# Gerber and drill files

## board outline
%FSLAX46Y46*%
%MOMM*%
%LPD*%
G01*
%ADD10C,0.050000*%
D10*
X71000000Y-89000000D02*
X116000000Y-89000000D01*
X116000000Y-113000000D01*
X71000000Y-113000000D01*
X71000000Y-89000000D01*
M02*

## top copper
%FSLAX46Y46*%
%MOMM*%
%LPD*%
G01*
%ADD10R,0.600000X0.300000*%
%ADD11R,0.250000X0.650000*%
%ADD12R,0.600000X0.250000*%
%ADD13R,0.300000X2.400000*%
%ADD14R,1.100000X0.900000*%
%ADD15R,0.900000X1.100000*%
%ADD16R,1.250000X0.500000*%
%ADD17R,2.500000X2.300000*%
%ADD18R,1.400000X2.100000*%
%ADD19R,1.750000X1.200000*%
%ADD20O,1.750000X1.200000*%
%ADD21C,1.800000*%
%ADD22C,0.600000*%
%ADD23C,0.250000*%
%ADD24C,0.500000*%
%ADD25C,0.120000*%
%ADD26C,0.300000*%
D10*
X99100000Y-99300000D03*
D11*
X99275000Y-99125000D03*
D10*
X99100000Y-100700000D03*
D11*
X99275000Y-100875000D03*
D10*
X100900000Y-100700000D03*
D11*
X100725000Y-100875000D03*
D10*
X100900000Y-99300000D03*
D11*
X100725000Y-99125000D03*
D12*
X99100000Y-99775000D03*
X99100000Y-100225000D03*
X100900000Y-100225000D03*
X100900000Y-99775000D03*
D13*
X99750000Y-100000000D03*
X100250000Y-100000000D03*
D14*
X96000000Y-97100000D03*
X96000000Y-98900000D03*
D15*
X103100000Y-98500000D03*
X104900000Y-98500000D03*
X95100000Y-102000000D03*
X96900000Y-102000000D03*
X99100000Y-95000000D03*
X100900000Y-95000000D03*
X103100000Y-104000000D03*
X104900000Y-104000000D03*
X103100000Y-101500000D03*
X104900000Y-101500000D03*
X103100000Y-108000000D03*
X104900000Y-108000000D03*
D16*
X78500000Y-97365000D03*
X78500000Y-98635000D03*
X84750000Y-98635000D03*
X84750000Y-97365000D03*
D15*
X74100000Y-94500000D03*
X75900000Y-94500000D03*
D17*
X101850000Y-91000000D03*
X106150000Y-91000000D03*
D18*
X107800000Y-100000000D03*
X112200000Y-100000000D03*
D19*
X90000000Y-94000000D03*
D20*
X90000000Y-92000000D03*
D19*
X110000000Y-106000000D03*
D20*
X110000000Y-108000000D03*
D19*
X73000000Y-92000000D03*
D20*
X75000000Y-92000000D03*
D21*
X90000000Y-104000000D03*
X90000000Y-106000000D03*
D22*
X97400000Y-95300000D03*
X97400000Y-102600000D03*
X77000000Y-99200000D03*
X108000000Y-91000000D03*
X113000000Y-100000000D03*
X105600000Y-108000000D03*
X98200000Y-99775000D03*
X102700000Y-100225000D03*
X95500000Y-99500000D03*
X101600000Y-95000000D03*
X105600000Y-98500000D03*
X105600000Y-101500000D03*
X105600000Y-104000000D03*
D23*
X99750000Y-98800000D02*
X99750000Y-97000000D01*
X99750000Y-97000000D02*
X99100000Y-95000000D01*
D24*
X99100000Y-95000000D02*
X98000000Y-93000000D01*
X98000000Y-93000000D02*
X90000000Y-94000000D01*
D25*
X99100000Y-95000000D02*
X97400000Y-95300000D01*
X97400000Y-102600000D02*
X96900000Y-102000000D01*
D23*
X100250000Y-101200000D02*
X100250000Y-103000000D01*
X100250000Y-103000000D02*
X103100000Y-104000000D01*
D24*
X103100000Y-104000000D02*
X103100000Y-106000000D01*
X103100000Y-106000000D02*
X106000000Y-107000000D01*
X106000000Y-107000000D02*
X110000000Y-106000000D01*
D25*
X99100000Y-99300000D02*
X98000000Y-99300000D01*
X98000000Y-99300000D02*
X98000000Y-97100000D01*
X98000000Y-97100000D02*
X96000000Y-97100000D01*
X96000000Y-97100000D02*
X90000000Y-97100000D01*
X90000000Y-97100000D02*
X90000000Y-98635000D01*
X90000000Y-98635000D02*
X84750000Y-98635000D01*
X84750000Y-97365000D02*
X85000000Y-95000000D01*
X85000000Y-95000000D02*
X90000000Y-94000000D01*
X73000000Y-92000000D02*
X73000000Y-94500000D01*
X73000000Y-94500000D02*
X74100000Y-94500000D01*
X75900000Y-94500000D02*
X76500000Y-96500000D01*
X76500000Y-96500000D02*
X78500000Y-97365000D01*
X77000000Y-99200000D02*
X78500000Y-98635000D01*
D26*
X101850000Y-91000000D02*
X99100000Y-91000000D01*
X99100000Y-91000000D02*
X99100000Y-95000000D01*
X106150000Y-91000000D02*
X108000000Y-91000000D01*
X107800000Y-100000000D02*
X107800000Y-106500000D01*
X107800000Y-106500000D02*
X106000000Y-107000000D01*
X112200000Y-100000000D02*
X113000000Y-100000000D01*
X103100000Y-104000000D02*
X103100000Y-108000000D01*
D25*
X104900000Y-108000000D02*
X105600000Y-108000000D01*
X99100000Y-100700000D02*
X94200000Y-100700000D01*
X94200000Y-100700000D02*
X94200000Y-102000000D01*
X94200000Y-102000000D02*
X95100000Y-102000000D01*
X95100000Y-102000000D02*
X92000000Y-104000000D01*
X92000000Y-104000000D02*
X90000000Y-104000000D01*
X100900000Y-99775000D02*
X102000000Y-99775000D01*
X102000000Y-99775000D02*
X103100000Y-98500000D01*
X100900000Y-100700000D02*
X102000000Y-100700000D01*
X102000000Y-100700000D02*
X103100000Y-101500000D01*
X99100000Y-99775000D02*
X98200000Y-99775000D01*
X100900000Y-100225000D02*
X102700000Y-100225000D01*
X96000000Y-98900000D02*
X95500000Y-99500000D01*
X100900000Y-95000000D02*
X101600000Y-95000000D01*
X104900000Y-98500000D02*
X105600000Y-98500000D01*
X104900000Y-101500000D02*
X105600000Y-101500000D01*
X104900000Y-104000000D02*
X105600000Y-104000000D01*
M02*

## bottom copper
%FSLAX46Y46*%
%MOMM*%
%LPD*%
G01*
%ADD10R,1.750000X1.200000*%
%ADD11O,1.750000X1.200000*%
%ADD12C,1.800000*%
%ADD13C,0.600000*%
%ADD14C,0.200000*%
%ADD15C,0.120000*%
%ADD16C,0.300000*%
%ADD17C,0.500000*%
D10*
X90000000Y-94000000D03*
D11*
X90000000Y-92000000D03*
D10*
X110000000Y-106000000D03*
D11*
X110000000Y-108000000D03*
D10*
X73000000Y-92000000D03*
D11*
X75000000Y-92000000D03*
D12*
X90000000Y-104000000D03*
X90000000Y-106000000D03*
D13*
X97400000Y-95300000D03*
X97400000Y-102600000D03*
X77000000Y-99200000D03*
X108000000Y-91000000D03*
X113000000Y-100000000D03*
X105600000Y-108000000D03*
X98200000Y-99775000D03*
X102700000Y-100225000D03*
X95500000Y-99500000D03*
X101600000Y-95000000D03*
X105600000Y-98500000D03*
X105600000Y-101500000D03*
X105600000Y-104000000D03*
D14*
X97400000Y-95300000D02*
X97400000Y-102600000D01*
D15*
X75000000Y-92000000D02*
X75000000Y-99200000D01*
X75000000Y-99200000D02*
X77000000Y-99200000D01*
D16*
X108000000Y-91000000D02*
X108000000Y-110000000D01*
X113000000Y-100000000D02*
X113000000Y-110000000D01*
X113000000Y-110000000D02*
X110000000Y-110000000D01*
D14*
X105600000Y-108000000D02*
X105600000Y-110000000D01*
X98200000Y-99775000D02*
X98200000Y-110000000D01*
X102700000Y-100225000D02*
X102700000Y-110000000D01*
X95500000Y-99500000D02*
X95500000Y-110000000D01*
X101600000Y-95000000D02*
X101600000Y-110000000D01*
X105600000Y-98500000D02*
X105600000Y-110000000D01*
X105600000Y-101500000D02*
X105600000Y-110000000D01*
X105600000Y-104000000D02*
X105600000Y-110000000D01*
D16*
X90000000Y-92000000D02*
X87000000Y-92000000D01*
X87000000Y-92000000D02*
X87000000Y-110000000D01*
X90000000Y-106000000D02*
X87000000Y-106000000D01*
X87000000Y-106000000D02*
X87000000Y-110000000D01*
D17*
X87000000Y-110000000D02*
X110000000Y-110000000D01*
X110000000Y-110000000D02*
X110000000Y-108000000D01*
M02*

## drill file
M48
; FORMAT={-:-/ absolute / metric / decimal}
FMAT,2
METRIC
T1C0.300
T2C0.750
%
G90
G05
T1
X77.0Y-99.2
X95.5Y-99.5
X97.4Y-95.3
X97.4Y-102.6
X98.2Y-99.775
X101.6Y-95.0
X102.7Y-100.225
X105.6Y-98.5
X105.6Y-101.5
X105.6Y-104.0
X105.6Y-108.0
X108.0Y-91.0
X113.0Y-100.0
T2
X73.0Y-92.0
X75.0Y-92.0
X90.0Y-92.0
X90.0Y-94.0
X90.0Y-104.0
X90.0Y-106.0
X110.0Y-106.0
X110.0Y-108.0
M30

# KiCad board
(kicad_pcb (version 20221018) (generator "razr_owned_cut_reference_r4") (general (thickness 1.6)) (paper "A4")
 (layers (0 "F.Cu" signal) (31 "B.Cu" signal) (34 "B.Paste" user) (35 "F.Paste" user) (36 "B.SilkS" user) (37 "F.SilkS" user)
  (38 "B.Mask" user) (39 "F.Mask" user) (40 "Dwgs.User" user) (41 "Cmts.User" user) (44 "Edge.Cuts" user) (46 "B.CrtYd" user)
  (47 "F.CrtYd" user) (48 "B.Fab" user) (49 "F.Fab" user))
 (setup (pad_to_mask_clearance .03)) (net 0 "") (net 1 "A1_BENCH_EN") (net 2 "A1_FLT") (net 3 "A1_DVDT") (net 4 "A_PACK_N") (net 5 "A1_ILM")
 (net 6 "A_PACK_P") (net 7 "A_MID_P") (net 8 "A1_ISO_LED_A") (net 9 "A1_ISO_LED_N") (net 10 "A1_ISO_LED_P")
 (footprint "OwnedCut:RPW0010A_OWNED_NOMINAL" (layer "F.Cu") (at 100 100)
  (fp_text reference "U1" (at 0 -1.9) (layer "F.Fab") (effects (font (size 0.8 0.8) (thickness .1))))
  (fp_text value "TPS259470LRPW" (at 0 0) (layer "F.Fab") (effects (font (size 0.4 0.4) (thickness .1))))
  (pad "1" smd rect (at -0.9 -0.7) (size 0.6 0.3) (layers "F.Cu" "F.Paste" "F.Mask") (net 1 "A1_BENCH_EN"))
  (pad "1" smd rect (at -0.725 -0.875) (size 0.25 0.65) (layers "F.Cu" "F.Paste" "F.Mask") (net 1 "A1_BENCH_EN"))
  (pad "4" smd rect (at -0.9 0.7) (size 0.6 0.3) (layers "F.Cu" "F.Paste" "F.Mask") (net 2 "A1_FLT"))
  (pad "4" smd rect (at -0.725 0.875) (size 0.25 0.65) (layers "F.Cu" "F.Paste" "F.Mask") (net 2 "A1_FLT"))
  (pad "7" smd rect (at 0.9 0.7) (size 0.6 0.3) (layers "F.Cu" "F.Paste" "F.Mask") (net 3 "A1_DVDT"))
  (pad "7" smd rect (at 0.725 0.875) (size 0.25 0.65) (layers "F.Cu" "F.Paste" "F.Mask") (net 3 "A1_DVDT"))
  (pad "10" smd rect (at 0.9 -0.7) (size 0.6 0.3) (layers "F.Cu" "F.Paste" "F.Mask"))
  (pad "10" smd rect (at 0.725 -0.875) (size 0.25 0.65) (layers "F.Cu" "F.Paste" "F.Mask"))
  (pad "2" smd rect (at -0.9 -0.225) (size 0.6 0.25) (layers "F.Cu" "F.Paste" "F.Mask") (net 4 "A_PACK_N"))
  (pad "3" smd rect (at -0.9 0.225) (size 0.6 0.25) (layers "F.Cu" "F.Paste" "F.Mask"))
  (pad "8" smd rect (at 0.9 0.225) (size 0.6 0.25) (layers "F.Cu" "F.Paste" "F.Mask") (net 4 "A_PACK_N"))
  (pad "9" smd rect (at 0.9 -0.225) (size 0.6 0.25) (layers "F.Cu" "F.Paste" "F.Mask") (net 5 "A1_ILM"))
  (pad "5" smd rect (at -0.25 0) (size 0.3 2.4) (layers "F.Cu" "F.Paste" "F.Mask") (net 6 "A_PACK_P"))
  (pad "6" smd rect (at 0.25 0) (size 0.3 2.4) (layers "F.Cu" "F.Paste" "F.Mask") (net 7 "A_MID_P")))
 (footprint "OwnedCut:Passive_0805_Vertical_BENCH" (layer "F.Cu") (at 96 98)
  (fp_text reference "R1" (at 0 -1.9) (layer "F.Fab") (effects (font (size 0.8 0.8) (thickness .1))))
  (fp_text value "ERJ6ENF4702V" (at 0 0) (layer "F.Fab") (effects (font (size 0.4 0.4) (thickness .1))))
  (pad "1" smd rect (at 0 -0.9) (size 1.1 0.9) (layers "F.Cu" "F.Paste" "F.Mask") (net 1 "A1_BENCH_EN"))
  (pad "2" smd rect (at 0 0.9) (size 1.1 0.9) (layers "F.Cu" "F.Paste" "F.Mask") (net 4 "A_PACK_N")))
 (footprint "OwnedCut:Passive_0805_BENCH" (layer "F.Cu") (at 104 98.5)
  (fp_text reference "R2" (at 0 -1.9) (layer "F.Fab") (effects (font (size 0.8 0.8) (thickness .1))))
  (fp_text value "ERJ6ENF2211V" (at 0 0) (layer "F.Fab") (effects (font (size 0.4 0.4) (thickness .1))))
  (pad "1" smd rect (at -0.9 0) (size 0.9 1.1) (layers "F.Cu" "F.Paste" "F.Mask") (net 5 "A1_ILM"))
  (pad "2" smd rect (at 0.9 0) (size 0.9 1.1) (layers "F.Cu" "F.Paste" "F.Mask") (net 4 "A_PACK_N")))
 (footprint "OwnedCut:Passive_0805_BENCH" (layer "F.Cu") (at 96 102)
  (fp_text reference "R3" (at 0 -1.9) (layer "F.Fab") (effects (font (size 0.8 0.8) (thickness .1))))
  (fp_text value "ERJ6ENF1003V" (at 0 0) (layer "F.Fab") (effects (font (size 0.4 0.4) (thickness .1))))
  (pad "1" smd rect (at -0.9 0) (size 0.9 1.1) (layers "F.Cu" "F.Paste" "F.Mask") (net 2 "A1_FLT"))
  (pad "2" smd rect (at 0.9 0) (size 0.9 1.1) (layers "F.Cu" "F.Paste" "F.Mask") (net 6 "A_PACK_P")))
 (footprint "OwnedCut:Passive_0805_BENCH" (layer "F.Cu") (at 100 95)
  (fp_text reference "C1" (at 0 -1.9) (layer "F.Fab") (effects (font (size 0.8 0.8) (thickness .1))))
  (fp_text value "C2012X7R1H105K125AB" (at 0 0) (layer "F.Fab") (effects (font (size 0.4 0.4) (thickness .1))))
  (pad "1" smd rect (at -0.9 0) (size 0.9 1.1) (layers "F.Cu" "F.Paste" "F.Mask") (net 6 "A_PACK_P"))
  (pad "2" smd rect (at 0.9 0) (size 0.9 1.1) (layers "F.Cu" "F.Paste" "F.Mask") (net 4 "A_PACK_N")))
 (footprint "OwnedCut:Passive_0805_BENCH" (layer "F.Cu") (at 104 104)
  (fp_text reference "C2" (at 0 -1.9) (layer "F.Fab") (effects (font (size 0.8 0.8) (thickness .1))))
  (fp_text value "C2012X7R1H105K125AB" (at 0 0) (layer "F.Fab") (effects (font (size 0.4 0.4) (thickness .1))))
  (pad "1" smd rect (at -0.9 0) (size 0.9 1.1) (layers "F.Cu" "F.Paste" "F.Mask") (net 7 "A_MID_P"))
  (pad "2" smd rect (at 0.9 0) (size 0.9 1.1) (layers "F.Cu" "F.Paste" "F.Mask") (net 4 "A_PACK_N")))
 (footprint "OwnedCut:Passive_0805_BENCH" (layer "F.Cu") (at 104 101.5)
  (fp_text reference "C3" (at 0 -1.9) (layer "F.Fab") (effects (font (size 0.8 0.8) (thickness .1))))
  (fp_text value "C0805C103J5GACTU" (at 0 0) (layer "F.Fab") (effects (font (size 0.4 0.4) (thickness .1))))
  (pad "1" smd rect (at -0.9 0) (size 0.9 1.1) (layers "F.Cu" "F.Paste" "F.Mask") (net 3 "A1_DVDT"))
  (pad "2" smd rect (at 0.9 0) (size 0.9 1.1) (layers "F.Cu" "F.Paste" "F.Mask") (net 4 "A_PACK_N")))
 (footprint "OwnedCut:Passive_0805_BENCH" (layer "F.Cu") (at 104 108)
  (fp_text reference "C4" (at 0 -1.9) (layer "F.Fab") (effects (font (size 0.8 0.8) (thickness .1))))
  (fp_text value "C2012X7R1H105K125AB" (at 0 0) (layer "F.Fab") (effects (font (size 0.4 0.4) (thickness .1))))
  (pad "1" smd rect (at -0.9 0) (size 0.9 1.1) (layers "F.Cu" "F.Paste" "F.Mask") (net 7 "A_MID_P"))
  (pad "2" smd rect (at 0.9 0) (size 0.9 1.1) (layers "F.Cu" "F.Paste" "F.Mask") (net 4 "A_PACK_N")))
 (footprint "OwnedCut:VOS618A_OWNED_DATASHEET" (layer "F.Cu") (at 81.625 98)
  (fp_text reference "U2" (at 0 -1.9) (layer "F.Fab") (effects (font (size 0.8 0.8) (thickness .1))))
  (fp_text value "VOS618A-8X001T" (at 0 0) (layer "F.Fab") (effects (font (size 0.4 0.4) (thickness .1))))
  (pad "1" smd rect (at -3.125 -0.635) (size 1.25 0.5) (layers "F.Cu" "F.Paste" "F.Mask") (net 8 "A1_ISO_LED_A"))
  (pad "2" smd rect (at -3.125 0.635) (size 1.25 0.5) (layers "F.Cu" "F.Paste" "F.Mask") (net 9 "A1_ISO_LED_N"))
  (pad "3" smd rect (at 3.125 0.635) (size 1.25 0.5) (layers "F.Cu" "F.Paste" "F.Mask") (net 1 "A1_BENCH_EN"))
  (pad "4" smd rect (at 3.125 -0.635) (size 1.25 0.5) (layers "F.Cu" "F.Paste" "F.Mask") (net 6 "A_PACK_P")))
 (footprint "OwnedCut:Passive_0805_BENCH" (layer "F.Cu") (at 75 94.5)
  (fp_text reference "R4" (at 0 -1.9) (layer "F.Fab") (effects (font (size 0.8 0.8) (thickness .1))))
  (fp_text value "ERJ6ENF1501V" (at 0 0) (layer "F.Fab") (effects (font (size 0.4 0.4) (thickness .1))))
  (pad "1" smd rect (at -0.9 0) (size 0.9 1.1) (layers "F.Cu" "F.Paste" "F.Mask") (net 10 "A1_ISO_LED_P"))
  (pad "2" smd rect (at 0.9 0) (size 0.9 1.1) (layers "F.Cu" "F.Paste" "F.Mask") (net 8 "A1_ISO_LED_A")))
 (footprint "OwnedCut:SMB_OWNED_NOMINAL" (layer "F.Cu") (at 104 91)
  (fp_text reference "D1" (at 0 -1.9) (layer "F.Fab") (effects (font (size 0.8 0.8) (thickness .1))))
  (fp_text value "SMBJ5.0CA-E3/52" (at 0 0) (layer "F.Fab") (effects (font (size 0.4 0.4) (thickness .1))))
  (pad "1" smd rect (at -2.15 0) (size 2.5 2.3) (layers "F.Cu" "F.Paste" "F.Mask") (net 6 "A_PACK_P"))
  (pad "2" smd rect (at 2.15 0) (size 2.5 2.3) (layers "F.Cu" "F.Paste" "F.Mask") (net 4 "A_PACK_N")))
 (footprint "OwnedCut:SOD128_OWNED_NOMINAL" (layer "F.Cu") (at 110 100)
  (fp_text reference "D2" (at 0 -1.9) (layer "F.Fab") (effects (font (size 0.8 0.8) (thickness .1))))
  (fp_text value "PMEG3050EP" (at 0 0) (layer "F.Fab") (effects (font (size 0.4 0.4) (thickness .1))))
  (pad "1" smd rect (at -2.2 0) (size 1.4 2.1) (layers "F.Cu" "F.Paste" "F.Mask") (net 7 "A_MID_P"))
  (pad "2" smd rect (at 2.2 0) (size 1.4 2.1) (layers "F.Cu" "F.Paste" "F.Mask") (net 4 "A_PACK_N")))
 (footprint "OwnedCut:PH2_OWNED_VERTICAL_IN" (layer "F.Cu") (at 90 94)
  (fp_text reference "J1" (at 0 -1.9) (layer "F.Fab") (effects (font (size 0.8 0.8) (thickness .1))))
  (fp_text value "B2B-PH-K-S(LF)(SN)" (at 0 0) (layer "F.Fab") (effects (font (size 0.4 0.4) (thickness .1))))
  (pad "1" thru_hole rect (at 0 0) (size 1.75 1.2) (drill .75) (layers "*.Cu" "*.Mask") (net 6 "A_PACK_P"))
  (pad "2" thru_hole oval (at 0 -2) (size 1.75 1.2) (drill .75) (layers "*.Cu" "*.Mask") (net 4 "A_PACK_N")))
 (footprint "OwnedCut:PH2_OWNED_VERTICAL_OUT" (layer "F.Cu") (at 110 106)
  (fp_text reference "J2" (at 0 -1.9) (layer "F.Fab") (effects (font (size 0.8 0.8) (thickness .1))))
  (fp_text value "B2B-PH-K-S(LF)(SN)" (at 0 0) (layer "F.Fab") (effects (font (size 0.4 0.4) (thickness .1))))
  (pad "1" thru_hole rect (at 0 0) (size 1.75 1.2) (drill .75) (layers "*.Cu" "*.Mask") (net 7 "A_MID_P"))
  (pad "2" thru_hole oval (at 0 2) (size 1.75 1.2) (drill .75) (layers "*.Cu" "*.Mask") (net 4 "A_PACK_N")))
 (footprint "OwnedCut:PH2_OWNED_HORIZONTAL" (layer "F.Cu") (at 73 92)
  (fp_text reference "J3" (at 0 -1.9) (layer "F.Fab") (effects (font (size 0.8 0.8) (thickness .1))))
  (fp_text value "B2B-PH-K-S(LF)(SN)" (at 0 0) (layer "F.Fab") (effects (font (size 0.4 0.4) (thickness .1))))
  (pad "1" thru_hole rect (at 0 0) (size 1.75 1.2) (drill .75) (layers "*.Cu" "*.Mask") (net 10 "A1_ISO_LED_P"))
  (pad "2" thru_hole oval (at 2 0) (size 1.75 1.2) (drill .75) (layers "*.Cu" "*.Mask") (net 9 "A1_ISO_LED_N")))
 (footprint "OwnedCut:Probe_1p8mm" (layer "F.Cu") (at 90 104)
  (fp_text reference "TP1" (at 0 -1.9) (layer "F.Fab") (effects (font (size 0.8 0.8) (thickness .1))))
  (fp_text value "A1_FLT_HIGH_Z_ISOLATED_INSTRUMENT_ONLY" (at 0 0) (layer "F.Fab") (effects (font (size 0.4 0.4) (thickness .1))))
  (pad "1" thru_hole circle (at 0 0) (size 1.8 1.8) (drill .75) (layers "*.Cu" "*.Mask") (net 2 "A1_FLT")))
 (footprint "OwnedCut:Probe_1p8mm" (layer "F.Cu") (at 90 106)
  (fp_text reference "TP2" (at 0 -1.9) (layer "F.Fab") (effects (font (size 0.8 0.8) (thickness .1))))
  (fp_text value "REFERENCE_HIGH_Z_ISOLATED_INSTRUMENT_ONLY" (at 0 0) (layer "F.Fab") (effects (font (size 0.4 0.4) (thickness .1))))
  (pad "1" thru_hole circle (at 0 0) (size 1.8 1.8) (drill .75) (layers "*.Cu" "*.Mask") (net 4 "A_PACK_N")))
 (segment (start 99.75 98.8) (end 99.75 97) (width 0.25) (layer "F.Cu") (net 6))
 (segment (start 99.75 97) (end 99.1 95) (width 0.25) (layer "F.Cu") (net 6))
 (segment (start 99.1 95) (end 98 93) (width 0.5) (layer "F.Cu") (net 6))
 (segment (start 98 93) (end 90 94) (width 0.5) (layer "F.Cu") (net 6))
 (segment (start 99.1 95) (end 97.4 95.3) (width 0.12) (layer "F.Cu") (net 6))
 (via (at 97.4 95.3) (size .6) (drill .3) (layers "F.Cu" "B.Cu") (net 6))
 (segment (start 97.4 95.3) (end 97.4 102.6) (width 0.2) (layer "B.Cu") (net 6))
 (via (at 97.4 102.6) (size .6) (drill .3) (layers "F.Cu" "B.Cu") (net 6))
 (segment (start 97.4 102.6) (end 96.9 102) (width 0.12) (layer "F.Cu") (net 6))
 (segment (start 100.25 101.2) (end 100.25 103) (width 0.25) (layer "F.Cu") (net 7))
 (segment (start 100.25 103) (end 103.1 104) (width 0.25) (layer "F.Cu") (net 7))
 (segment (start 103.1 104) (end 103.1 106) (width 0.5) (layer "F.Cu") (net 7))
 (segment (start 103.1 106) (end 106 107) (width 0.5) (layer "F.Cu") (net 7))
 (segment (start 106 107) (end 110 106) (width 0.5) (layer "F.Cu") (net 7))
 (segment (start 99.1 99.3) (end 98 99.3) (width 0.12) (layer "F.Cu") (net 1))
 (segment (start 98 99.3) (end 98 97.1) (width 0.12) (layer "F.Cu") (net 1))
 (segment (start 98 97.1) (end 96 97.1) (width 0.12) (layer "F.Cu") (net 1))
 (segment (start 96 97.1) (end 90 97.1) (width 0.12) (layer "F.Cu") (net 1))
 (segment (start 90 97.1) (end 90 98.635) (width 0.12) (layer "F.Cu") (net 1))
 (segment (start 90 98.635) (end 84.75 98.635) (width 0.12) (layer "F.Cu") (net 1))
 (segment (start 84.75 97.365) (end 85 95) (width 0.12) (layer "F.Cu") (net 6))
 (segment (start 85 95) (end 90 94) (width 0.12) (layer "F.Cu") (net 6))
 (segment (start 73 92) (end 73 94.5) (width 0.12) (layer "F.Cu") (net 10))
 (segment (start 73 94.5) (end 74.1 94.5) (width 0.12) (layer "F.Cu") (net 10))
 (segment (start 75.9 94.5) (end 76.5 96.5) (width 0.12) (layer "F.Cu") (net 8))
 (segment (start 76.5 96.5) (end 78.5 97.365) (width 0.12) (layer "F.Cu") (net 8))
 (segment (start 75 92) (end 75 99.2) (width 0.12) (layer "B.Cu") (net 9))
 (segment (start 75 99.2) (end 77 99.2) (width 0.12) (layer "B.Cu") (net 9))
 (via (at 77 99.2) (size .6) (drill .3) (layers "F.Cu" "B.Cu") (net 9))
 (segment (start 77 99.2) (end 78.5 98.635) (width 0.12) (layer "F.Cu") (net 9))
 (segment (start 101.85 91) (end 99.1 91) (width 0.3) (layer "F.Cu") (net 6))
 (segment (start 99.1 91) (end 99.1 95) (width 0.3) (layer "F.Cu") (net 6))
 (segment (start 106.15 91) (end 108 91) (width 0.3) (layer "F.Cu") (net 4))
 (via (at 108 91) (size .6) (drill .3) (layers "F.Cu" "B.Cu") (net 4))
 (segment (start 108 91) (end 108 110) (width 0.3) (layer "B.Cu") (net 4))
 (segment (start 107.8 100) (end 107.8 106.5) (width 0.3) (layer "F.Cu") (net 7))
 (segment (start 107.8 106.5) (end 106 107) (width 0.3) (layer "F.Cu") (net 7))
 (segment (start 112.2 100) (end 113 100) (width 0.3) (layer "F.Cu") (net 4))
 (via (at 113 100) (size .6) (drill .3) (layers "F.Cu" "B.Cu") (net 4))
 (segment (start 113 100) (end 113 110) (width 0.3) (layer "B.Cu") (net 4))
 (segment (start 113 110) (end 110 110) (width 0.3) (layer "B.Cu") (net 4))
 (segment (start 103.1 104) (end 103.1 108) (width 0.3) (layer "F.Cu") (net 7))
 (segment (start 104.9 108) (end 105.6 108) (width 0.12) (layer "F.Cu") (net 4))
 (via (at 105.6 108) (size .6) (drill .3) (layers "F.Cu" "B.Cu") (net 4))
 (segment (start 105.6 108) (end 105.6 110) (width 0.2) (layer "B.Cu") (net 4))
 (segment (start 99.1 100.7) (end 94.2 100.7) (width 0.12) (layer "F.Cu") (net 2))
 (segment (start 94.2 100.7) (end 94.2 102) (width 0.12) (layer "F.Cu") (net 2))
 (segment (start 94.2 102) (end 95.1 102) (width 0.12) (layer "F.Cu") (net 2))
 (segment (start 95.1 102) (end 92 104) (width 0.12) (layer "F.Cu") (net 2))
 (segment (start 92 104) (end 90 104) (width 0.12) (layer "F.Cu") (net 2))
 (segment (start 100.9 99.775) (end 102 99.775) (width 0.12) (layer "F.Cu") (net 5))
 (segment (start 102 99.775) (end 103.1 98.5) (width 0.12) (layer "F.Cu") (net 5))
 (segment (start 100.9 100.7) (end 102 100.7) (width 0.12) (layer "F.Cu") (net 3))
 (segment (start 102 100.7) (end 103.1 101.5) (width 0.12) (layer "F.Cu") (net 3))
 (segment (start 99.1 99.775) (end 98.2 99.775) (width 0.12) (layer "F.Cu") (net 4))
 (via (at 98.2 99.775) (size .6) (drill .3) (layers "F.Cu" "B.Cu") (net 4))
 (segment (start 98.2 99.775) (end 98.2 110) (width 0.2) (layer "B.Cu") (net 4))
 (segment (start 100.9 100.225) (end 102.7 100.225) (width 0.12) (layer "F.Cu") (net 4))
 (via (at 102.7 100.225) (size .6) (drill .3) (layers "F.Cu" "B.Cu") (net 4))
 (segment (start 102.7 100.225) (end 102.7 110) (width 0.2) (layer "B.Cu") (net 4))
 (segment (start 96 98.9) (end 95.5 99.5) (width 0.12) (layer "F.Cu") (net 4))
 (via (at 95.5 99.5) (size .6) (drill .3) (layers "F.Cu" "B.Cu") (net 4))
 (segment (start 95.5 99.5) (end 95.5 110) (width 0.2) (layer "B.Cu") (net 4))
 (segment (start 100.9 95) (end 101.6 95) (width 0.12) (layer "F.Cu") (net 4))
 (via (at 101.6 95) (size .6) (drill .3) (layers "F.Cu" "B.Cu") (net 4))
 (segment (start 101.6 95) (end 101.6 110) (width 0.2) (layer "B.Cu") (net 4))
 (segment (start 104.9 98.5) (end 105.6 98.5) (width 0.12) (layer "F.Cu") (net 4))
 (via (at 105.6 98.5) (size .6) (drill .3) (layers "F.Cu" "B.Cu") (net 4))
 (segment (start 105.6 98.5) (end 105.6 110) (width 0.2) (layer "B.Cu") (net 4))
 (segment (start 104.9 101.5) (end 105.6 101.5) (width 0.12) (layer "F.Cu") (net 4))
 (via (at 105.6 101.5) (size .6) (drill .3) (layers "F.Cu" "B.Cu") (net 4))
 (segment (start 105.6 101.5) (end 105.6 110) (width 0.2) (layer "B.Cu") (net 4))
 (segment (start 104.9 104) (end 105.6 104) (width 0.12) (layer "F.Cu") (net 4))
 (via (at 105.6 104) (size .6) (drill .3) (layers "F.Cu" "B.Cu") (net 4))
 (segment (start 105.6 104) (end 105.6 110) (width 0.2) (layer "B.Cu") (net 4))
 (segment (start 90 92) (end 87 92) (width 0.3) (layer "B.Cu") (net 4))
 (segment (start 87 92) (end 87 110) (width 0.3) (layer "B.Cu") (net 4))
 (segment (start 90 106) (end 87 106) (width 0.3) (layer "B.Cu") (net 4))
 (segment (start 87 106) (end 87 110) (width 0.3) (layer "B.Cu") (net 4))
 (segment (start 87 110) (end 110 110) (width 0.5) (layer "B.Cu") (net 4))
 (segment (start 110 110) (end 110 108) (width 0.5) (layer "B.Cu") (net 4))
 (gr_rect (start 71 89) (end 116 113) (stroke (width .05) (type default)) (fill none) (layer "Edge.Cuts")))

